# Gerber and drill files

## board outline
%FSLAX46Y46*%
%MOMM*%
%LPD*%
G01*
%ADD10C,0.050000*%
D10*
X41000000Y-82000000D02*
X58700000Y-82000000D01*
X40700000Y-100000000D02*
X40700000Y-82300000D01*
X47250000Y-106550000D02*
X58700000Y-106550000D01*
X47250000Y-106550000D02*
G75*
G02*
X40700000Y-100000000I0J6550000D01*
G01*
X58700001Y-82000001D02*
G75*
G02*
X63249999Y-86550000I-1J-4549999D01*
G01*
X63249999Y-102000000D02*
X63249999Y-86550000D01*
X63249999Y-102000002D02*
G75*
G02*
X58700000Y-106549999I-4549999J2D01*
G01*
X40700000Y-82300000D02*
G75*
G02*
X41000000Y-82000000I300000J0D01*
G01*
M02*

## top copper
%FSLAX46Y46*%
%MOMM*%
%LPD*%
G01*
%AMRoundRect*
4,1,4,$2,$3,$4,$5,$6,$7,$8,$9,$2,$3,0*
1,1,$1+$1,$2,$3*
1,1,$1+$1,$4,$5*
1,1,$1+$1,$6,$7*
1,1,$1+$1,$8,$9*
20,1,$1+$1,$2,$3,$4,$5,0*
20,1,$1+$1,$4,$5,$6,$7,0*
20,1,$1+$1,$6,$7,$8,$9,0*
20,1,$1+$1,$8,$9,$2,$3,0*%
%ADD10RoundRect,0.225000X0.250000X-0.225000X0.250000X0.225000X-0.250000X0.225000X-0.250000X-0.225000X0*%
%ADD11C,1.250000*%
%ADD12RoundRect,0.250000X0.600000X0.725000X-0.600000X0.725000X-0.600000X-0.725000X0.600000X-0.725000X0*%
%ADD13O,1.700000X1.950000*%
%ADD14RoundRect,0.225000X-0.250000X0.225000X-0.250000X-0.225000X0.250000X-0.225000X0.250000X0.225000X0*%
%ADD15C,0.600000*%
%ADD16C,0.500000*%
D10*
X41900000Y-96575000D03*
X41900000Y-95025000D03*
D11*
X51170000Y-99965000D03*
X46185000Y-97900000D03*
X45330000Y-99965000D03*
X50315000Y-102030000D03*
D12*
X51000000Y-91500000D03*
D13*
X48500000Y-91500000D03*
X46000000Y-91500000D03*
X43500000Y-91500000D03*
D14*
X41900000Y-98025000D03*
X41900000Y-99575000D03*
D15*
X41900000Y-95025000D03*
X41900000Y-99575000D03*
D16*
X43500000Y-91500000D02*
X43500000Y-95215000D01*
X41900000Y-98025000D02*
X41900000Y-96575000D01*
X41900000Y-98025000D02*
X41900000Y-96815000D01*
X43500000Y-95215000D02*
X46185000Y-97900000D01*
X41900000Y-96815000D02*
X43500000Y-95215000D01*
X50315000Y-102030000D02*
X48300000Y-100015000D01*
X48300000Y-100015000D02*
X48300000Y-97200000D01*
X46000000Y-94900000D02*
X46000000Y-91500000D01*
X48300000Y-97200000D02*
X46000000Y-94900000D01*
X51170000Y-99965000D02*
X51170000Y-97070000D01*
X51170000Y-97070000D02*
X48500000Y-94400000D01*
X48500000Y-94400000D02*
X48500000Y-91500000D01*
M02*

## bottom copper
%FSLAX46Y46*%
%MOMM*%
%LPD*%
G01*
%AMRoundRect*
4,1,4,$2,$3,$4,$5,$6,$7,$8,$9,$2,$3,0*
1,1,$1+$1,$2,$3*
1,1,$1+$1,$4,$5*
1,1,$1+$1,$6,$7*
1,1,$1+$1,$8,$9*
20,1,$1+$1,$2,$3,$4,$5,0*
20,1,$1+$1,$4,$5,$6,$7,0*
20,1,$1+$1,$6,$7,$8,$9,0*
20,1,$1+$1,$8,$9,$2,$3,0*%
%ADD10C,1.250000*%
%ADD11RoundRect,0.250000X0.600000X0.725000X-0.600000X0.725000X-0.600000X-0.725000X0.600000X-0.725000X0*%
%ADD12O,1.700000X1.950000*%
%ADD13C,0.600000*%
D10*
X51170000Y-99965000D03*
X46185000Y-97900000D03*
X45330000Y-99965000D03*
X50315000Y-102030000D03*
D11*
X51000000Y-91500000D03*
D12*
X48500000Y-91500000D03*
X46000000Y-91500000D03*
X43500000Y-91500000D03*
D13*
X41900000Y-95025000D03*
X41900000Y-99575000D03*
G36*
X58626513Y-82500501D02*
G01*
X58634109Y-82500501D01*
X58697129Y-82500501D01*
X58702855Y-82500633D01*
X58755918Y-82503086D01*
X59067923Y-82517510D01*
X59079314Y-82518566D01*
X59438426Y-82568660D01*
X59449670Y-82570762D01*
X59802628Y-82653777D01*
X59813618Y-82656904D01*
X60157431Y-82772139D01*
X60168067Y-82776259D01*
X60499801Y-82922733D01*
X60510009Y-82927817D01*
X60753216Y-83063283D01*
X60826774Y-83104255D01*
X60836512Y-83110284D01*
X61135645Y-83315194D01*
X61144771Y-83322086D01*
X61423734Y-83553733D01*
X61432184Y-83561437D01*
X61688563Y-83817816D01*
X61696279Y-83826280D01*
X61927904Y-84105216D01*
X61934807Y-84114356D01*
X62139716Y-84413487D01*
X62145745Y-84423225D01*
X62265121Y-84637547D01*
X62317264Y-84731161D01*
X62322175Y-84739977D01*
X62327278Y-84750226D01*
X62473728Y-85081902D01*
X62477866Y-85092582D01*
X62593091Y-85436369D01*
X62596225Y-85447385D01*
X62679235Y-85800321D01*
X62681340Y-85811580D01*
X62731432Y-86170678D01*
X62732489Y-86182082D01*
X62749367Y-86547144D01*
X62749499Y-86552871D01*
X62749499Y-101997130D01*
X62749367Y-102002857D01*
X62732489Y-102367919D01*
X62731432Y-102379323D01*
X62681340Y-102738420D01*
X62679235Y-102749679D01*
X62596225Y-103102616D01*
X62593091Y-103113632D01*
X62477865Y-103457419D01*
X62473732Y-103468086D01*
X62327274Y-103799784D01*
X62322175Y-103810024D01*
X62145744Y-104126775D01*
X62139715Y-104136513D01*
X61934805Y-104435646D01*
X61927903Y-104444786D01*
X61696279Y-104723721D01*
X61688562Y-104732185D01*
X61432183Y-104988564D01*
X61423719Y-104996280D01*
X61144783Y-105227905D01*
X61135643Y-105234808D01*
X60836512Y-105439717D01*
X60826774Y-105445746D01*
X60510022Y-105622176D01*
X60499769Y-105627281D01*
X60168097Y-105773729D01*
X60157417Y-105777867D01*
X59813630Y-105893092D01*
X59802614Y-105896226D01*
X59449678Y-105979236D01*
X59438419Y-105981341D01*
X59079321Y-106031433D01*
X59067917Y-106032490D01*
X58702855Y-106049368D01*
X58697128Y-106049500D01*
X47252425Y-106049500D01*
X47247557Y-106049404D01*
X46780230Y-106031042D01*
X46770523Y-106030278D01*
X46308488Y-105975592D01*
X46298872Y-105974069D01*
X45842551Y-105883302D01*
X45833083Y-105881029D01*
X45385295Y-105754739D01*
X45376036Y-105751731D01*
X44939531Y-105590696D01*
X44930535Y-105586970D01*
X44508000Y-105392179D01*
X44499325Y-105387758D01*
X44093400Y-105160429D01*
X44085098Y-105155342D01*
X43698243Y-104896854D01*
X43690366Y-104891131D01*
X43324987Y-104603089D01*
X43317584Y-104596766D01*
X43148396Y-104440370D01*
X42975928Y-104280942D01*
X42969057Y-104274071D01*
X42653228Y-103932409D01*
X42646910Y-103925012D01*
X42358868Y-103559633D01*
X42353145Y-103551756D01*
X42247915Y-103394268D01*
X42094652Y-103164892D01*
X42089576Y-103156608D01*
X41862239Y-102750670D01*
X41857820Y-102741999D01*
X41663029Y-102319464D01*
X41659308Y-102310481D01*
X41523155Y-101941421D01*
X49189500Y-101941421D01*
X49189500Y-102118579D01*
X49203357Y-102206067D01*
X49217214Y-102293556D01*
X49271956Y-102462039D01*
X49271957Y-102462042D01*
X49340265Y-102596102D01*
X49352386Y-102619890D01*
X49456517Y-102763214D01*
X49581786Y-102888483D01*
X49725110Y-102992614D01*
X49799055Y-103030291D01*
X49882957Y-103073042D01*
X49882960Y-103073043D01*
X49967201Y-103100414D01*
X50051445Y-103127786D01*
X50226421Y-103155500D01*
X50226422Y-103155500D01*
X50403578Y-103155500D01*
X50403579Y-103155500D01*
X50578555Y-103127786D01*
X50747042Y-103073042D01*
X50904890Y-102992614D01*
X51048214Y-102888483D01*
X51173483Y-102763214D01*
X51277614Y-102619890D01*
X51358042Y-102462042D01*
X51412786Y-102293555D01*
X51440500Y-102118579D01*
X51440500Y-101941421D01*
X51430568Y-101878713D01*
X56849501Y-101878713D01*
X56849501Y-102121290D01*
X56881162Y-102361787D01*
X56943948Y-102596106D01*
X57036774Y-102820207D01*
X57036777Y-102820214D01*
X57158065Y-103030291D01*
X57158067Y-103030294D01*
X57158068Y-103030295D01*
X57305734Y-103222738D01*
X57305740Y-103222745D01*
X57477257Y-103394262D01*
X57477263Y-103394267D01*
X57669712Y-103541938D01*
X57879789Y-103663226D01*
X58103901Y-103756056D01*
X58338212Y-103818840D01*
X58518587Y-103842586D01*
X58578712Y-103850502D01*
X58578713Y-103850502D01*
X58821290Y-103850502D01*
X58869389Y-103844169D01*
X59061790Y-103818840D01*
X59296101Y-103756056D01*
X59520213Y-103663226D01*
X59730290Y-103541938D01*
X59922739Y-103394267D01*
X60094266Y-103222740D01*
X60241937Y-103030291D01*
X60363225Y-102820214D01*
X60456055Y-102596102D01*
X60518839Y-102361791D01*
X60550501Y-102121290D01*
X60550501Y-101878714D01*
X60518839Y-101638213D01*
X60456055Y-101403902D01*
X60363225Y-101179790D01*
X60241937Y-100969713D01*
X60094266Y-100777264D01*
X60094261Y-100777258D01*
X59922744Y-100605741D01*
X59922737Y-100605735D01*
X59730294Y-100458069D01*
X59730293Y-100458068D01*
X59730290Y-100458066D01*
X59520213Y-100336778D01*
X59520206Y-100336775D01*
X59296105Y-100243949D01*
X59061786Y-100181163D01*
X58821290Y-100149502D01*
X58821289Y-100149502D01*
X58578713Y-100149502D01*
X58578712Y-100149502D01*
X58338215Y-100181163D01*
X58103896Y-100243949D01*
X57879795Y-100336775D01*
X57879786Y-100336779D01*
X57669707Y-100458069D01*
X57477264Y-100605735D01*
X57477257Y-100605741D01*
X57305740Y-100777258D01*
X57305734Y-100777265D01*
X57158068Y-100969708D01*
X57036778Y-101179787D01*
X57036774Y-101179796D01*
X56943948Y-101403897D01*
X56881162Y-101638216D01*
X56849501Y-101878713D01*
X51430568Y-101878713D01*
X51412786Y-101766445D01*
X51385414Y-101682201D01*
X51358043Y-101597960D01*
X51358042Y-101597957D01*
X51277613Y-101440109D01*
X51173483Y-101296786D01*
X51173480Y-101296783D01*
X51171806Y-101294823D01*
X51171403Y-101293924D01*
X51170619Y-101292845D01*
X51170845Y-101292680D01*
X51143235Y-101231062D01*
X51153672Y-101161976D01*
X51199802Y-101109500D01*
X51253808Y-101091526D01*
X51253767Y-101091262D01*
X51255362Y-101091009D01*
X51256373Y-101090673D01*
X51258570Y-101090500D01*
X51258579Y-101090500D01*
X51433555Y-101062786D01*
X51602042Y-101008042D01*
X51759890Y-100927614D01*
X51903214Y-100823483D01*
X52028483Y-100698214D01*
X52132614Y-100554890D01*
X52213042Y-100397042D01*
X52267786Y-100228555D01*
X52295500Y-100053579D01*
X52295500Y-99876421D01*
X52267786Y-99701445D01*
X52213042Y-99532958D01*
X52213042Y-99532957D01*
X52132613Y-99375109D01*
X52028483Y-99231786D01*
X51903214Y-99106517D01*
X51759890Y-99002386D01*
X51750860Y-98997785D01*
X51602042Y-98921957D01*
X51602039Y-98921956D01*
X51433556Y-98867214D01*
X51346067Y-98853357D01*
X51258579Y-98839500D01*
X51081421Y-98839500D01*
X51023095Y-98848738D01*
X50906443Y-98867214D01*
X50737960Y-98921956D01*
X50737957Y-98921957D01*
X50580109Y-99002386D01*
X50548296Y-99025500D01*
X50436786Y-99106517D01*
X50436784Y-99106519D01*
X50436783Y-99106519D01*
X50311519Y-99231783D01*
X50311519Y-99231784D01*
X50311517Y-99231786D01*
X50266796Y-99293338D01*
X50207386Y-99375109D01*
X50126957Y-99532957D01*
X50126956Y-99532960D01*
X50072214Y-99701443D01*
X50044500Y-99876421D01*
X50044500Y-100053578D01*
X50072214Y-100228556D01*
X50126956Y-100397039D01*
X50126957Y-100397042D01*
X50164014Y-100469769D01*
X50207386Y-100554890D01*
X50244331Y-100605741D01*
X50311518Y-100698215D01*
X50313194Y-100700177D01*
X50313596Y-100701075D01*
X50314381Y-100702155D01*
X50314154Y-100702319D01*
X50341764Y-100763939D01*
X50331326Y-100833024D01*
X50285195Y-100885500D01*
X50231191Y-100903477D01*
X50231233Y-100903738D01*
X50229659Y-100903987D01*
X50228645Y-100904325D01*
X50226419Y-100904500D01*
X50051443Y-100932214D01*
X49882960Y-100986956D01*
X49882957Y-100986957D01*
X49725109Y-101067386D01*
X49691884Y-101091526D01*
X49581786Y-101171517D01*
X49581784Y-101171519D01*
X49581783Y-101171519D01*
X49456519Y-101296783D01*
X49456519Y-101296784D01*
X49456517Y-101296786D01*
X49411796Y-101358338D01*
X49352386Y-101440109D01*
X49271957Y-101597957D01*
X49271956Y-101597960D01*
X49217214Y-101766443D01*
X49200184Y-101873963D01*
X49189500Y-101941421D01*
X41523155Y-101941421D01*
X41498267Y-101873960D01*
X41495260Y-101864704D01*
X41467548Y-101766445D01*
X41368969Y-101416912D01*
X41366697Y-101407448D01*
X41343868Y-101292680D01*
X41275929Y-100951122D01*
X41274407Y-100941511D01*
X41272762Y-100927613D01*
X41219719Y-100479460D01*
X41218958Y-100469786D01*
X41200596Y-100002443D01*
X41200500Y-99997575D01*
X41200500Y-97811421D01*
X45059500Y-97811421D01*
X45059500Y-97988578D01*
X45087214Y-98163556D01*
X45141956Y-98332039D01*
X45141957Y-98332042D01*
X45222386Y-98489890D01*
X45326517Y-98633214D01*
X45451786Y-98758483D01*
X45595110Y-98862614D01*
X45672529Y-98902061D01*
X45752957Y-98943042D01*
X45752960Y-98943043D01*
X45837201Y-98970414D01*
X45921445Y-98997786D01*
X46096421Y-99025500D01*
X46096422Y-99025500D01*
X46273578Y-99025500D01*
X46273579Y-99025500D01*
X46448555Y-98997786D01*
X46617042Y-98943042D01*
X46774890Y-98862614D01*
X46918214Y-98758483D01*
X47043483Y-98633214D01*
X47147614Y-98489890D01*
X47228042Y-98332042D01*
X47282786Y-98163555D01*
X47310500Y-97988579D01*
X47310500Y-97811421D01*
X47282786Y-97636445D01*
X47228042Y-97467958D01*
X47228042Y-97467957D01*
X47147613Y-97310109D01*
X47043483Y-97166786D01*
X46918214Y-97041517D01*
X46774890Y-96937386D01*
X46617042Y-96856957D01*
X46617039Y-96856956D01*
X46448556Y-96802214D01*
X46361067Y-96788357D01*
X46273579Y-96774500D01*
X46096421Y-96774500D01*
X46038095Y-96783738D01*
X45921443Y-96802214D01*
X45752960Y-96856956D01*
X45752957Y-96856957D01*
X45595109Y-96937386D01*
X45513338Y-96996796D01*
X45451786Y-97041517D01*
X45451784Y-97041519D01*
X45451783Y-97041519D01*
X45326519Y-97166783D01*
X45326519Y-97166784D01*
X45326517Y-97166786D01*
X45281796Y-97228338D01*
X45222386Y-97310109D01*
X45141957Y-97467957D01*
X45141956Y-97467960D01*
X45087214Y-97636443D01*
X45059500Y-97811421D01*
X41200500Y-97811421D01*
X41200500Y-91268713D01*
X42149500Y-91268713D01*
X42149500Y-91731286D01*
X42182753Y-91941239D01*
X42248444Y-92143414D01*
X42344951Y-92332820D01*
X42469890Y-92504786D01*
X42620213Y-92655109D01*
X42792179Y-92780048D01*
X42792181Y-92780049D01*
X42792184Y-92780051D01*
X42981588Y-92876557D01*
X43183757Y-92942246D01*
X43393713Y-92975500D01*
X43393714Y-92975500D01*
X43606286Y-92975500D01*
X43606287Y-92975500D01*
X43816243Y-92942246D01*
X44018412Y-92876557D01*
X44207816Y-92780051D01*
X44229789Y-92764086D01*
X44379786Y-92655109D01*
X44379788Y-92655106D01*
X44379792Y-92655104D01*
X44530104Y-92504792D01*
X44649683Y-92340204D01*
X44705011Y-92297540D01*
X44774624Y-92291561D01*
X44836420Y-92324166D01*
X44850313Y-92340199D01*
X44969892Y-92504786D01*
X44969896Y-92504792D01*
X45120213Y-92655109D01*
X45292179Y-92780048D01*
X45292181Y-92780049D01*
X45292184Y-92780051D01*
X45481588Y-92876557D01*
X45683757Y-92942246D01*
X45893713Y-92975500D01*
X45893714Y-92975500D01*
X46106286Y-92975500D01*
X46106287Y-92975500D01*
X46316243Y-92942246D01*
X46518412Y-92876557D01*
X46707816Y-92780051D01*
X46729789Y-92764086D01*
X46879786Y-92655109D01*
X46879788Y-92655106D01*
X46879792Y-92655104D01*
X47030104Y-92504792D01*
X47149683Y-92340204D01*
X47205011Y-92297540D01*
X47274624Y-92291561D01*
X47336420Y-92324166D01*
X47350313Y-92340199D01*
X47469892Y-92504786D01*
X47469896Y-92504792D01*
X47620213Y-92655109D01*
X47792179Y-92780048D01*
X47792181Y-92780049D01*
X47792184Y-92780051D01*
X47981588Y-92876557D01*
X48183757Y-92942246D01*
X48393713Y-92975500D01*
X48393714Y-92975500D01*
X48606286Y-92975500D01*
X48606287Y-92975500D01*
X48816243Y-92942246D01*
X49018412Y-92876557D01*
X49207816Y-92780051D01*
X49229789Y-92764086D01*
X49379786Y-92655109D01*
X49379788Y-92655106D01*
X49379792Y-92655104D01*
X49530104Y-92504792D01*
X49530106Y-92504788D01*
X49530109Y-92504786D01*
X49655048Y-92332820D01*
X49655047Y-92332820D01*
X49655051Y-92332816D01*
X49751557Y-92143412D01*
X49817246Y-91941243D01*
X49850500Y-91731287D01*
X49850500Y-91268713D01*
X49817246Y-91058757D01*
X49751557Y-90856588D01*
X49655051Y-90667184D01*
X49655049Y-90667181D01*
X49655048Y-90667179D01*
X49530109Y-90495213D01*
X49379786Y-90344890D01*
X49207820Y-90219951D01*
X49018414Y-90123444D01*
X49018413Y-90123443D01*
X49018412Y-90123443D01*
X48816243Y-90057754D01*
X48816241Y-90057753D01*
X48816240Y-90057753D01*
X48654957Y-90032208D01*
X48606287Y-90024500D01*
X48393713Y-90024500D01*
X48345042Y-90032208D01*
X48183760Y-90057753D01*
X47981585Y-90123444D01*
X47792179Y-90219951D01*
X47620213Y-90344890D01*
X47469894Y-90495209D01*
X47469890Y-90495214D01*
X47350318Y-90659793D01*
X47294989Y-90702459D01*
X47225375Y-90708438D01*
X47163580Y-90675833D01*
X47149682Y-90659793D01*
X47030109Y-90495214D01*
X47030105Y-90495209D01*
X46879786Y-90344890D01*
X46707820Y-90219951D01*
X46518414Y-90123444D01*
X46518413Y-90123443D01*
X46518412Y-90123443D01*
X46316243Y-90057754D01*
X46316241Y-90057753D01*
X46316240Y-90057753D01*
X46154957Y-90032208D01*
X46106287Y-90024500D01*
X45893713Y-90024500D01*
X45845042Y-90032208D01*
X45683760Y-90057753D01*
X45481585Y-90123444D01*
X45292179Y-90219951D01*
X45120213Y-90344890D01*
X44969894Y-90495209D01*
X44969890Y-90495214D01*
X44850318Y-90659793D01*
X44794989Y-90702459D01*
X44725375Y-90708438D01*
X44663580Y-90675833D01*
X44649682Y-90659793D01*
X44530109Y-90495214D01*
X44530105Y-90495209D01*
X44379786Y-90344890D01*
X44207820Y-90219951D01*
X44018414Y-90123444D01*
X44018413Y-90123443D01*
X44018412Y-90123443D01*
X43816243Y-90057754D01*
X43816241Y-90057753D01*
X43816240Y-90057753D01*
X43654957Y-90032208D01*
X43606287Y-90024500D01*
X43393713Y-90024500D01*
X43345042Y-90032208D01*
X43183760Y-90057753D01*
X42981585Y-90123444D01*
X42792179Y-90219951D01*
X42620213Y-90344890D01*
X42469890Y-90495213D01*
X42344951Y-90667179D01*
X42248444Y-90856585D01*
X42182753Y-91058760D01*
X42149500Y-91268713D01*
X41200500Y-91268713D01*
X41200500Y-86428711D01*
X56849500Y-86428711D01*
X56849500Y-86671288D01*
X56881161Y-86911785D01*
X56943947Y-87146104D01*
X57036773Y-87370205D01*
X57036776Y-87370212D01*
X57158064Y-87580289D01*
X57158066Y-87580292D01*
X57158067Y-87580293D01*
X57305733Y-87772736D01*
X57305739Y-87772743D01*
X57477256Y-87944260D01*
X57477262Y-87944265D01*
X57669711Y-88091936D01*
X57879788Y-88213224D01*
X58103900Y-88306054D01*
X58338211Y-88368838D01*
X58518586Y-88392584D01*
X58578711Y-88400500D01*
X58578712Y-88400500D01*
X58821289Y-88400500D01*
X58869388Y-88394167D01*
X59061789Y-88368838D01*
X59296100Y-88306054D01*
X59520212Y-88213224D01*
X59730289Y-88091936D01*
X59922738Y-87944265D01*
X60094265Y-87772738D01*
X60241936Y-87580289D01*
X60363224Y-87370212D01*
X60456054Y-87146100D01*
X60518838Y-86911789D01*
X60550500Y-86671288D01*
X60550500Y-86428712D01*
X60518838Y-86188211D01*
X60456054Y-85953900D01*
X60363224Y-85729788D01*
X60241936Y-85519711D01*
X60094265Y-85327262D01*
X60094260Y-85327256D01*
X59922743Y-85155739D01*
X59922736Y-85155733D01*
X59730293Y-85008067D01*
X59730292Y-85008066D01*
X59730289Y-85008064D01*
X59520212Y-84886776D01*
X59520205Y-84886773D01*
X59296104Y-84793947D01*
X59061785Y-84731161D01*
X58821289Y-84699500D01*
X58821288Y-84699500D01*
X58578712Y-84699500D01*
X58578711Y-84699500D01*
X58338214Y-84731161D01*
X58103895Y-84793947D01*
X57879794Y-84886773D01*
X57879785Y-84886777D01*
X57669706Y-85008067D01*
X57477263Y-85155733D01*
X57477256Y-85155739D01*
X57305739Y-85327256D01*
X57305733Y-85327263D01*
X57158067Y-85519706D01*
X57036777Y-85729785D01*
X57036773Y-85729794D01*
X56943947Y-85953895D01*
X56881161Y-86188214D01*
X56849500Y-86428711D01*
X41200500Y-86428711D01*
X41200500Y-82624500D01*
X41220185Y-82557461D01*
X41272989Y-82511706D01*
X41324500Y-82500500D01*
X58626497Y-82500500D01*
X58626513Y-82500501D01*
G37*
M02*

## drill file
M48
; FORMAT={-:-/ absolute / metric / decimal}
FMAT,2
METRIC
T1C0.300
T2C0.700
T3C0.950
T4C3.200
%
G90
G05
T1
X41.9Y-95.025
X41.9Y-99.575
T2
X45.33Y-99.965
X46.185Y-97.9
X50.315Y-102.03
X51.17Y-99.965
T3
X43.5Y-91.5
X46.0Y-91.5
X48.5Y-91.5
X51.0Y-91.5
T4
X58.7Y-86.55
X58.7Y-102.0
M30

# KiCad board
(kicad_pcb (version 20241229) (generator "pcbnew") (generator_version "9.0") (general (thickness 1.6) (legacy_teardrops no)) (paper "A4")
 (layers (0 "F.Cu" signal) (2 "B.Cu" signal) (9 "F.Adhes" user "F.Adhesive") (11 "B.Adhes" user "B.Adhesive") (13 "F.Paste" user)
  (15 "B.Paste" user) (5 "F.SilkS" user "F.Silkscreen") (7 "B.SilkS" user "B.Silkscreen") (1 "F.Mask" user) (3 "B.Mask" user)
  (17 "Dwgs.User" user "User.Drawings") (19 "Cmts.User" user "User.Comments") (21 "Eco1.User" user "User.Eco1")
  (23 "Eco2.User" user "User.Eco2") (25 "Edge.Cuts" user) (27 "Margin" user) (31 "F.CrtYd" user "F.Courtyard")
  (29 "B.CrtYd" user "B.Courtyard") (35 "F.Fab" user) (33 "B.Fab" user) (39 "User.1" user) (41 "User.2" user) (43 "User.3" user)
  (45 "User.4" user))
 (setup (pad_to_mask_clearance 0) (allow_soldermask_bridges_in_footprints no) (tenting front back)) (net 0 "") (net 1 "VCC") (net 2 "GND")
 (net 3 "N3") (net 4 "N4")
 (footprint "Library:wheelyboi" (layer "F.Cu") (at 61.05 89.3 -90)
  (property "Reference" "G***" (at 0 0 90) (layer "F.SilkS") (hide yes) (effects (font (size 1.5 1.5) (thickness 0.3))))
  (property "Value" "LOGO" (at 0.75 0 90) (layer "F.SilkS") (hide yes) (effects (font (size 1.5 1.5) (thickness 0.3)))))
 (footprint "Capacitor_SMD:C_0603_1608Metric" (layer "F.Cu") (at 41.9 95.8 90)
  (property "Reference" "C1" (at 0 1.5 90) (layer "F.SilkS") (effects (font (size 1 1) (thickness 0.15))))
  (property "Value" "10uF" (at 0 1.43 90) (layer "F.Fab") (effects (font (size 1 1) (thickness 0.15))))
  (pad "1" smd roundrect (at -0.775 0 90) (size 0.9 0.95) (layers "F.Cu" "F.Mask" "F.Paste") (roundrect_rratio 0.25) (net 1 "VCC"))
  (pad "2" smd roundrect (at 0.775 0 90) (size 0.9 0.95) (layers "F.Cu" "F.Mask" "F.Paste") (roundrect_rratio 0.25) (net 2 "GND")))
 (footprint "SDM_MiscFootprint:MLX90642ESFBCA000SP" (layer "F.Cu") (at 51.17 99.965 180)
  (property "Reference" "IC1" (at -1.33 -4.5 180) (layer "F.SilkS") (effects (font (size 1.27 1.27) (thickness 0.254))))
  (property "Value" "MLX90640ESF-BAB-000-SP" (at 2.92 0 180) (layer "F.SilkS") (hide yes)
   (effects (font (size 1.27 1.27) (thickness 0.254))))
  (pad "1" thru_hole circle (at 0 0 180) (size 1.25 1.25) (drill 0.7) (layers "*.Cu" "*.Mask") (remove_unused_layers no) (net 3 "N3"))
  (pad "2" thru_hole circle (at 4.985 2.065 180) (size 1.25 1.25) (drill 0.7) (layers "*.Cu" "*.Mask") (remove_unused_layers no)
   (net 1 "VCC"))
  (pad "3" thru_hole circle (at 5.84 0 180) (size 1.25 1.25) (drill 0.7) (layers "*.Cu" "*.Mask") (remove_unused_layers no) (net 2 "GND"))
  (pad "4" thru_hole circle (at 0.855 -2.065 180) (size 1.25 1.25) (drill 0.7) (layers "*.Cu" "*.Mask") (remove_unused_layers no)
   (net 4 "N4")))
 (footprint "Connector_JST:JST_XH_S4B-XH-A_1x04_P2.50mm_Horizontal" (layer "F.Cu") (at 51 91.5 180)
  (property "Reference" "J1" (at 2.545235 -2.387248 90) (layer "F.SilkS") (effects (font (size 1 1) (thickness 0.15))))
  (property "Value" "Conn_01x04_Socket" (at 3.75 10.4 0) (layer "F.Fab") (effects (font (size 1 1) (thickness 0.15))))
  (pad "1" thru_hole roundrect (at 0 0 180) (size 1.7 1.95) (drill 0.95) (layers "*.Cu" "*.Mask") (remove_unused_layers no)
   (roundrect_rratio 0.147059) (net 2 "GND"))
  (pad "2" thru_hole oval (at 2.5 0 180) (size 1.7 1.95) (drill 0.95) (layers "*.Cu" "*.Mask") (remove_unused_layers no) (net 3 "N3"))
  (pad "3" thru_hole oval (at 5 0 180) (size 1.7 1.95) (drill 0.95) (layers "*.Cu" "*.Mask") (remove_unused_layers no) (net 4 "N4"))
  (pad "4" thru_hole oval (at 7.5 0 180) (size 1.7 1.95) (drill 0.95) (layers "*.Cu" "*.Mask") (remove_unused_layers no) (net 1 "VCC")))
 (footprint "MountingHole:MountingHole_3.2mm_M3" (layer "F.Cu") (at 58.7 86.55)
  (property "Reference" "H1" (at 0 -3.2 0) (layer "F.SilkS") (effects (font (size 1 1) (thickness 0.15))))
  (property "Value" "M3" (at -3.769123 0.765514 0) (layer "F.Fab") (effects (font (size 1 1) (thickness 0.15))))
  (pad "" np_thru_hole circle (at 0 0) (size 3.2 3.2) (drill 3.2) (layers "*.Cu" "*.Mask")))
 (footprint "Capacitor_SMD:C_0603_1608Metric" (layer "F.Cu") (at 41.9 98.8 -90)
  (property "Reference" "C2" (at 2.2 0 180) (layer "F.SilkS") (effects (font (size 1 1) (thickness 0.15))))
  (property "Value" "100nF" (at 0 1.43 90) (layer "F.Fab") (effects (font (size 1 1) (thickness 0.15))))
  (pad "1" smd roundrect (at -0.775 0 270) (size 0.9 0.95) (layers "F.Cu" "F.Mask" "F.Paste") (roundrect_rratio 0.25) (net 1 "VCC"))
  (pad "2" smd roundrect (at 0.775 0 270) (size 0.9 0.95) (layers "F.Cu" "F.Mask" "F.Paste") (roundrect_rratio 0.25) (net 2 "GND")))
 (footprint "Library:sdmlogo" (layer "F.Cu") (at 62 95.3 -90)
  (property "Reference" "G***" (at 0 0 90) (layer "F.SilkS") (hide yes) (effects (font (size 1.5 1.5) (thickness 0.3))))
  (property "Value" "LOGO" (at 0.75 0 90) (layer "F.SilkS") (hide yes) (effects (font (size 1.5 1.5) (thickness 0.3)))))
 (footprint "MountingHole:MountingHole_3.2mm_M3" (layer "F.Cu") (at 58.700001 102.000002)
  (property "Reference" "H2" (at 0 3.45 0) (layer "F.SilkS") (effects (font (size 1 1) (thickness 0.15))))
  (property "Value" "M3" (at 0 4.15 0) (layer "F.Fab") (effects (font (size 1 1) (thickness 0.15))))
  (pad "" np_thru_hole circle (at 0 0) (size 3.2 3.2) (drill 3.2) (layers "*.Cu" "*.Mask")))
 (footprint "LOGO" (layer "B.Cu") (at 47.304066 85.596581 90)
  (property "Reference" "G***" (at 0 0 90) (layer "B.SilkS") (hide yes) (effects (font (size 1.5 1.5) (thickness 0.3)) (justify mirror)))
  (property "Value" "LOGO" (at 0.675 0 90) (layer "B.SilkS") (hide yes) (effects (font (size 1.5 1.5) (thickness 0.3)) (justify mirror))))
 (gr_line (start 41 82) (end 58.7 82) (stroke (width 0.05) (type default)) (layer "Edge.Cuts"))
 (gr_line (start 40.7 100) (end 40.7 82.3) (stroke (width 0.05) (type default)) (layer "Edge.Cuts"))
 (gr_line (start 47.25 106.55) (end 58.7 106.55) (stroke (width 0.05) (type default)) (layer "Edge.Cuts"))
 (gr_arc (start 47.25 106.55) (mid 42.618451 104.631549) (end 40.7 100) (stroke (width 0.05) (type solid)) (layer "Edge.Cuts"))
 (gr_arc (start 58.700001 82.000001) (mid 61.917336 83.332665) (end 63.249999 86.55) (stroke (width 0.05) (type default))
  (layer "Edge.Cuts"))
 (gr_line (start 63.249999 102) (end 63.249999 86.55) (stroke (width 0.05) (type default)) (layer "Edge.Cuts"))
 (gr_arc (start 63.249999 102.000002) (mid 61.917335 105.217337) (end 58.7 106.55) (stroke (width 0.05) (type default)) (layer "Edge.Cuts"))
 (gr_arc (start 40.7 82.3) (mid 40.787868 82.087868) (end 41 82) (stroke (width 0.05) (type default)) (layer "Edge.Cuts"))
 (segment (start 43.5 91.5) (end 43.5 95.215) (width 0.5) (layer "F.Cu") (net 1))
 (segment (start 41.9 98.025) (end 41.9 96.575) (width 0.5) (layer "F.Cu") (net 1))
 (segment (start 41.9 98.025) (end 41.9 96.815) (width 0.5) (layer "F.Cu") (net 1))
 (segment (start 43.5 95.215) (end 46.185 97.9) (width 0.5) (layer "F.Cu") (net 1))
 (segment (start 41.9 96.815) (end 43.5 95.215) (width 0.5) (layer "F.Cu") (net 1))
 (segment (start 50.315 102.03) (end 48.3 100.015) (width 0.5) (layer "F.Cu") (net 4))
 (segment (start 48.3 100.015) (end 48.3 97.2) (width 0.5) (layer "F.Cu") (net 4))
 (segment (start 46 94.9) (end 46 91.5) (width 0.5) (layer "F.Cu") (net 4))
 (segment (start 48.3 97.2) (end 46 94.9) (width 0.5) (layer "F.Cu") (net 4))
 (via (at 41.9 95.025) (size 0.6) (drill 0.3) (layers "F.Cu" "B.Cu") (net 2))
 (via (at 41.9 99.575) (size 0.6) (drill 0.3) (layers "F.Cu" "B.Cu") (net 2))
 (segment (start 51.17 99.965) (end 51.17 97.07) (width 0.5) (layer "F.Cu") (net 3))
 (segment (start 51.17 97.07) (end 48.5 94.4) (width 0.5) (layer "F.Cu") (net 3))
 (segment (start 48.5 94.4) (end 48.5 91.5) (width 0.5) (layer "F.Cu") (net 3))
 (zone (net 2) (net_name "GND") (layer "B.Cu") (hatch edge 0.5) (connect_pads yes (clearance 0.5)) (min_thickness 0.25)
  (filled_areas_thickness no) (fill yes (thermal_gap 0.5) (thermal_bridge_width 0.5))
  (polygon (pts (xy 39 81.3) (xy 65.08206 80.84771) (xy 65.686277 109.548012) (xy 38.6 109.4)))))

